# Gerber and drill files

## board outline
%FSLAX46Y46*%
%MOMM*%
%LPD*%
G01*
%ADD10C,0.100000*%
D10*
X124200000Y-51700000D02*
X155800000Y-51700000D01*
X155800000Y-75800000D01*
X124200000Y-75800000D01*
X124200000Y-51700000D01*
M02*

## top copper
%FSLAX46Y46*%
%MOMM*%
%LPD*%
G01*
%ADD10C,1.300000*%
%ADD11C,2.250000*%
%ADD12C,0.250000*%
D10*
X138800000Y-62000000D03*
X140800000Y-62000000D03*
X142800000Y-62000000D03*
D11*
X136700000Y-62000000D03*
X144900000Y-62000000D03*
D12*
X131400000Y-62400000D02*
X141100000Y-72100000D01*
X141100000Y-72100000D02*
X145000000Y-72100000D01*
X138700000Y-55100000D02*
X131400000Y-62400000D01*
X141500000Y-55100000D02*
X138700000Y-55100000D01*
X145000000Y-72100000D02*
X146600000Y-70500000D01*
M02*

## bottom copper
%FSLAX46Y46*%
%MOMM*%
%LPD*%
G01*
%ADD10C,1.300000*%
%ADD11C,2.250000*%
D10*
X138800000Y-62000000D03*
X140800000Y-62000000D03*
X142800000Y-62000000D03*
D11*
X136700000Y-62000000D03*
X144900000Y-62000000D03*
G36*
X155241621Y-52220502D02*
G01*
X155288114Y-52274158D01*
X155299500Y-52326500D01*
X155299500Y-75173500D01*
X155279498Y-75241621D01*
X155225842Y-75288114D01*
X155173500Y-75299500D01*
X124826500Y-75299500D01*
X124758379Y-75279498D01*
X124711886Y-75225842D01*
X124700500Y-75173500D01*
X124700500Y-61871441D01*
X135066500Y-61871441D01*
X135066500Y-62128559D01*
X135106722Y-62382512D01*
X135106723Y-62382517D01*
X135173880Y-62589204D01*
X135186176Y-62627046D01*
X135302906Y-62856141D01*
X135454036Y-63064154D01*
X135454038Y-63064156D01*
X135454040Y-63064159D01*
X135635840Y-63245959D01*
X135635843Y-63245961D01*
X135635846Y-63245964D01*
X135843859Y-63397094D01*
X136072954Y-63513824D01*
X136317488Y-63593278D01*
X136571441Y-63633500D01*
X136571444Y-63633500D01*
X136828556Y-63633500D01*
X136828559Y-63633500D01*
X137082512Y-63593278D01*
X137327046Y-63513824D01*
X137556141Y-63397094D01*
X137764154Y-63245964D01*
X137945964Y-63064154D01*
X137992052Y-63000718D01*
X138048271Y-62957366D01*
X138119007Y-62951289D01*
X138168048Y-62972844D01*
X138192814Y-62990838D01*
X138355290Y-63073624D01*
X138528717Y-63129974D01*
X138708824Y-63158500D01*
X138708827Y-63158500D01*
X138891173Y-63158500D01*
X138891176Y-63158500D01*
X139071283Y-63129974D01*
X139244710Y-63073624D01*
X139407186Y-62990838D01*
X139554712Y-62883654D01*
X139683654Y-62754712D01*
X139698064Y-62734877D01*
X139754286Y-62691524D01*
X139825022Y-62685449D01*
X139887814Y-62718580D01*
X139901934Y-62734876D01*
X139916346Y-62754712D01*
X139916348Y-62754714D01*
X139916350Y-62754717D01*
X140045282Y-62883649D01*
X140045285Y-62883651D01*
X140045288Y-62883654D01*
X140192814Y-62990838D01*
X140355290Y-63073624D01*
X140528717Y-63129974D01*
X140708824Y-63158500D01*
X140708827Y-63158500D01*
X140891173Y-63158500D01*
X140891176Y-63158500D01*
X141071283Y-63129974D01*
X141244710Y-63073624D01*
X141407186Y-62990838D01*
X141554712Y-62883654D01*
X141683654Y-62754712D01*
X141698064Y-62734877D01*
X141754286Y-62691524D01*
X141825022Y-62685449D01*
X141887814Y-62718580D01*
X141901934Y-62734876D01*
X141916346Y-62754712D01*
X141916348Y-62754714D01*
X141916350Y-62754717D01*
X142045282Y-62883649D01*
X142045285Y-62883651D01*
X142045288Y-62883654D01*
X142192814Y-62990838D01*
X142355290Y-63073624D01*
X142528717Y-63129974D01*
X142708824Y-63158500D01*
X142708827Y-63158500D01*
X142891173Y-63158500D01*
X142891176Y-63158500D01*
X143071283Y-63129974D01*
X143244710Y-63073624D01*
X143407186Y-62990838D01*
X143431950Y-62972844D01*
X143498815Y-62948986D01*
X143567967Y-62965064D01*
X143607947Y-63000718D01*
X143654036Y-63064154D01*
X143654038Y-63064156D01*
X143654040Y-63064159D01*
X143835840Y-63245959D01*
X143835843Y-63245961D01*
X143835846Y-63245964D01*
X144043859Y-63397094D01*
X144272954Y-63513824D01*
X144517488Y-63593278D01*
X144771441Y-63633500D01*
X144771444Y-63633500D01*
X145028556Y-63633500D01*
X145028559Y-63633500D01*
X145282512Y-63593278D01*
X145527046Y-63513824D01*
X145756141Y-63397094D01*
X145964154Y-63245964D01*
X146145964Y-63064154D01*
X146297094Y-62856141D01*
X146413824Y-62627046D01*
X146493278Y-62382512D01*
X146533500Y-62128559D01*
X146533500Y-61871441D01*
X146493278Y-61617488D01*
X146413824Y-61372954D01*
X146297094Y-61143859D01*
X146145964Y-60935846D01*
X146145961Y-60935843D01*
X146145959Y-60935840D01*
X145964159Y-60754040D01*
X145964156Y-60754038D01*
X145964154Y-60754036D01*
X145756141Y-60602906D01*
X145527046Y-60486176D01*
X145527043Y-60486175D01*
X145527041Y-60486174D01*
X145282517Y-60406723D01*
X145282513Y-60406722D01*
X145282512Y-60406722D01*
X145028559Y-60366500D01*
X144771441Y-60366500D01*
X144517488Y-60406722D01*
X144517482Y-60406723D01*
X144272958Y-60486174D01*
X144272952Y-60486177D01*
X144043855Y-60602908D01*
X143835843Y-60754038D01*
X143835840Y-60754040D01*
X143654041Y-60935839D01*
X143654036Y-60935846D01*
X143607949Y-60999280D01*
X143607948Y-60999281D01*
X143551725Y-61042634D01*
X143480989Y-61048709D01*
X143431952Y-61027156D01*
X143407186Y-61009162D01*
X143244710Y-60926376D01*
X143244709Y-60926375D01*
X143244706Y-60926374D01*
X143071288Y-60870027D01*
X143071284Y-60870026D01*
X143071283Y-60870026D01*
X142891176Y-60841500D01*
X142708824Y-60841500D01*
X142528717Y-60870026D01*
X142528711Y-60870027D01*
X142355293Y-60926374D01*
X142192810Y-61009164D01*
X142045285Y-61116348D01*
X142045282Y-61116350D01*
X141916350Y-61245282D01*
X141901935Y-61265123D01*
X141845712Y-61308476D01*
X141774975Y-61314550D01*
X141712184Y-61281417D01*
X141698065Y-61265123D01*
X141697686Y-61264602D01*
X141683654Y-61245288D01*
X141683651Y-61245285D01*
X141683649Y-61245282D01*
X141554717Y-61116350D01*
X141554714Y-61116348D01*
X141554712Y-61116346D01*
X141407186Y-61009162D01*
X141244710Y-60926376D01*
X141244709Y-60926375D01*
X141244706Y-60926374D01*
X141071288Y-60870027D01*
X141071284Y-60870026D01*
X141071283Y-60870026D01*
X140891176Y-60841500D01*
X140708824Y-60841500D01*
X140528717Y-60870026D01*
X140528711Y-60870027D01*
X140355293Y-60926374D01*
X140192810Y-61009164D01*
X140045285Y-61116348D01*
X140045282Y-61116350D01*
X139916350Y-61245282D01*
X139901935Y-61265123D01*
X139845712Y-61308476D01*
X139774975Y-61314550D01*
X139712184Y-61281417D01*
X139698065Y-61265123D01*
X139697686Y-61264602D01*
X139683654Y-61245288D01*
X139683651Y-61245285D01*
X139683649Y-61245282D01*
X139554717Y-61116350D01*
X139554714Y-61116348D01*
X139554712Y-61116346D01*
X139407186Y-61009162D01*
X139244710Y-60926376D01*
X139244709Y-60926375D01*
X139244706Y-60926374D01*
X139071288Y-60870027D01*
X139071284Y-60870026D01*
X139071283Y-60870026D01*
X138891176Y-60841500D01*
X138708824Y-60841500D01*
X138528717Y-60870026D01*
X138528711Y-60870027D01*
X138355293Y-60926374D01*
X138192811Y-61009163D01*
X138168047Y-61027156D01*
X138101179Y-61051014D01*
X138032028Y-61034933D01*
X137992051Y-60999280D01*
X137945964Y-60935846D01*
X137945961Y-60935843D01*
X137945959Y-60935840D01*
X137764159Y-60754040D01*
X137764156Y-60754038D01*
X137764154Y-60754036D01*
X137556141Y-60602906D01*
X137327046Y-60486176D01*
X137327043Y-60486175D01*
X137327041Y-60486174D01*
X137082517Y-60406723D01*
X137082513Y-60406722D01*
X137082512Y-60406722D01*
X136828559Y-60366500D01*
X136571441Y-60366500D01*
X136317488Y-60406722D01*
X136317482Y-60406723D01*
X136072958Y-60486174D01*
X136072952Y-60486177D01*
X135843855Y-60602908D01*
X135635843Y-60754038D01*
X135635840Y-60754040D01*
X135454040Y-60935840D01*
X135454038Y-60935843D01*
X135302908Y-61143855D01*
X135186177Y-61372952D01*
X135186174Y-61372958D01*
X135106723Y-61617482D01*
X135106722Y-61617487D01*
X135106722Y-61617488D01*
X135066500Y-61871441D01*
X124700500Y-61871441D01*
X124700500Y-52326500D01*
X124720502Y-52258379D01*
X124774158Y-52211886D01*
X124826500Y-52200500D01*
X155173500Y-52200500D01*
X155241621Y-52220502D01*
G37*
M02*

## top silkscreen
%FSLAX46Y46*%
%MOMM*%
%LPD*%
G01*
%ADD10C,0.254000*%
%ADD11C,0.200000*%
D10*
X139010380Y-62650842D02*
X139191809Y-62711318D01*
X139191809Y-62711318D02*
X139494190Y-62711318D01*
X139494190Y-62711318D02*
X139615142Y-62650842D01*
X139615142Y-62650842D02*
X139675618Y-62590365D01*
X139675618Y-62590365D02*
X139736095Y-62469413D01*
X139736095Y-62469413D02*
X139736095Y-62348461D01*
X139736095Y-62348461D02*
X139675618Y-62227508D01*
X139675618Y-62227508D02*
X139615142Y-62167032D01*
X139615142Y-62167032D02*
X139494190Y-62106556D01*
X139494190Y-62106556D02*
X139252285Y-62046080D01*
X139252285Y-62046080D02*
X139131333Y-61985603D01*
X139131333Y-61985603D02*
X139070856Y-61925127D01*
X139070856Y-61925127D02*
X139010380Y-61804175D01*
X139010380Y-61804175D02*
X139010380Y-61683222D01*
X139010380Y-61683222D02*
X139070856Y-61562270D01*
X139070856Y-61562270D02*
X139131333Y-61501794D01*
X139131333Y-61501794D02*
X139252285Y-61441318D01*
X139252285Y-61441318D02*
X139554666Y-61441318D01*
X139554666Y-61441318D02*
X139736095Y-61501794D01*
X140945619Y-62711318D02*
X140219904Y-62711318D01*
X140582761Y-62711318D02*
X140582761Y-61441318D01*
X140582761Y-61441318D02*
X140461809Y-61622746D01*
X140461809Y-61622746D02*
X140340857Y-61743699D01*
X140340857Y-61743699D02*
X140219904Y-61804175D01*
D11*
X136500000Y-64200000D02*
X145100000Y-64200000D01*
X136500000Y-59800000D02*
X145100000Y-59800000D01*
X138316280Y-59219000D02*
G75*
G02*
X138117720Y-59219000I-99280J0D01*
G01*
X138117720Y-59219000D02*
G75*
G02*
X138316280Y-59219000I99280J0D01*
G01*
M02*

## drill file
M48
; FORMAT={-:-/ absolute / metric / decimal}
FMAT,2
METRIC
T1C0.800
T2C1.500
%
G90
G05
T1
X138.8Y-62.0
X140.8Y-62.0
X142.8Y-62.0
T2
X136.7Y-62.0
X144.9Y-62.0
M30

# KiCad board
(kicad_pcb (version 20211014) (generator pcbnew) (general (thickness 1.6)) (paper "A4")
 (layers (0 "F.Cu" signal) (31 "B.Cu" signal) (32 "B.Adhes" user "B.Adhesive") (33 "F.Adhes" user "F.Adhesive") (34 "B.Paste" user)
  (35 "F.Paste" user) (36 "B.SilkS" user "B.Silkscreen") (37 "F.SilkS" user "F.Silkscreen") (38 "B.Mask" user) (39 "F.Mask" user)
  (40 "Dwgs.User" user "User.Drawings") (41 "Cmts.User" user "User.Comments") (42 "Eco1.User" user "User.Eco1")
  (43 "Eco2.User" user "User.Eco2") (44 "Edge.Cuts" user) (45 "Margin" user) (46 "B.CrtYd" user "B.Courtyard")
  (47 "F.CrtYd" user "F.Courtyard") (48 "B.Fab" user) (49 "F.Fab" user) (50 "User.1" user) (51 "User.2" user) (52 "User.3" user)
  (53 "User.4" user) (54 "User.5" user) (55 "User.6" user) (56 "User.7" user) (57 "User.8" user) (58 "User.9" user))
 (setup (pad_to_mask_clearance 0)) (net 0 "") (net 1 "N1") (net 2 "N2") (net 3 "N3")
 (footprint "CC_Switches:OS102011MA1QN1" (layer "F.Cu") (at 140.8 62)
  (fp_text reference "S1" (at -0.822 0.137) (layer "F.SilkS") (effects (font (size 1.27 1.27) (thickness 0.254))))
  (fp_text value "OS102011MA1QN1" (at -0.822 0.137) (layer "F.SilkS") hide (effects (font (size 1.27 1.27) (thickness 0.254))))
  (fp_line (start -4.3 2.2) (end 4.3 2.2) (layer "F.SilkS") (width 0.2))
  (fp_line (start -4.3 -2.2) (end 4.3 -2.2) (layer "F.SilkS") (width 0.2))
  (fp_circle (center -2.583 -2.781) (end -2.583 -2.68172) (layer "F.SilkS") (width 0.2) (fill none))
  (pad "1" thru_hole circle (at -2 0) (size 1.3 1.3) (drill 0.8) (layers *.Cu *.Mask) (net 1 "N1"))
  (pad "2" thru_hole circle (at 0 0) (size 1.3 1.3) (drill 0.8) (layers *.Cu *.Mask) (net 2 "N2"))
  (pad "3" thru_hole circle (at 2 0) (size 1.3 1.3) (drill 0.8) (layers *.Cu *.Mask) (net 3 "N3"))
  (pad "4" thru_hole circle (at -4.1 0) (size 2.25 2.25) (drill 1.5) (layers *.Cu *.Mask))
  (pad "5" thru_hole circle (at 4.1 0) (size 2.25 2.25) (drill 1.5) (layers *.Cu *.Mask)))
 (gr_rect (start 155.8 51.7) (end 124.2 75.8) (layer "Edge.Cuts") (width 0.1) (fill none))
 (segment (start 131.4 62.4) (end 141.1 72.1) (width 0.25) (layer "F.Cu") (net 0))
 (segment (start 141.1 72.1) (end 145 72.1) (width 0.25) (layer "F.Cu") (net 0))
 (segment (start 138.7 55.1) (end 131.4 62.4) (width 0.25) (layer "F.Cu") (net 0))
 (segment (start 141.5 55.1) (end 138.7 55.1) (width 0.25) (layer "F.Cu") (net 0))
 (segment (start 145 72.1) (end 146.6 70.5) (width 0.25) (layer "F.Cu") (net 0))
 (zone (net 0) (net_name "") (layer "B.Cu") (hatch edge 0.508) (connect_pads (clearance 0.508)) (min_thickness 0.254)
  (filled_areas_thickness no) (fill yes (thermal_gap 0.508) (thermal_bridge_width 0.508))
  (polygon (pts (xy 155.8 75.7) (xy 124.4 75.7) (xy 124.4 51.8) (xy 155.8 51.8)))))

